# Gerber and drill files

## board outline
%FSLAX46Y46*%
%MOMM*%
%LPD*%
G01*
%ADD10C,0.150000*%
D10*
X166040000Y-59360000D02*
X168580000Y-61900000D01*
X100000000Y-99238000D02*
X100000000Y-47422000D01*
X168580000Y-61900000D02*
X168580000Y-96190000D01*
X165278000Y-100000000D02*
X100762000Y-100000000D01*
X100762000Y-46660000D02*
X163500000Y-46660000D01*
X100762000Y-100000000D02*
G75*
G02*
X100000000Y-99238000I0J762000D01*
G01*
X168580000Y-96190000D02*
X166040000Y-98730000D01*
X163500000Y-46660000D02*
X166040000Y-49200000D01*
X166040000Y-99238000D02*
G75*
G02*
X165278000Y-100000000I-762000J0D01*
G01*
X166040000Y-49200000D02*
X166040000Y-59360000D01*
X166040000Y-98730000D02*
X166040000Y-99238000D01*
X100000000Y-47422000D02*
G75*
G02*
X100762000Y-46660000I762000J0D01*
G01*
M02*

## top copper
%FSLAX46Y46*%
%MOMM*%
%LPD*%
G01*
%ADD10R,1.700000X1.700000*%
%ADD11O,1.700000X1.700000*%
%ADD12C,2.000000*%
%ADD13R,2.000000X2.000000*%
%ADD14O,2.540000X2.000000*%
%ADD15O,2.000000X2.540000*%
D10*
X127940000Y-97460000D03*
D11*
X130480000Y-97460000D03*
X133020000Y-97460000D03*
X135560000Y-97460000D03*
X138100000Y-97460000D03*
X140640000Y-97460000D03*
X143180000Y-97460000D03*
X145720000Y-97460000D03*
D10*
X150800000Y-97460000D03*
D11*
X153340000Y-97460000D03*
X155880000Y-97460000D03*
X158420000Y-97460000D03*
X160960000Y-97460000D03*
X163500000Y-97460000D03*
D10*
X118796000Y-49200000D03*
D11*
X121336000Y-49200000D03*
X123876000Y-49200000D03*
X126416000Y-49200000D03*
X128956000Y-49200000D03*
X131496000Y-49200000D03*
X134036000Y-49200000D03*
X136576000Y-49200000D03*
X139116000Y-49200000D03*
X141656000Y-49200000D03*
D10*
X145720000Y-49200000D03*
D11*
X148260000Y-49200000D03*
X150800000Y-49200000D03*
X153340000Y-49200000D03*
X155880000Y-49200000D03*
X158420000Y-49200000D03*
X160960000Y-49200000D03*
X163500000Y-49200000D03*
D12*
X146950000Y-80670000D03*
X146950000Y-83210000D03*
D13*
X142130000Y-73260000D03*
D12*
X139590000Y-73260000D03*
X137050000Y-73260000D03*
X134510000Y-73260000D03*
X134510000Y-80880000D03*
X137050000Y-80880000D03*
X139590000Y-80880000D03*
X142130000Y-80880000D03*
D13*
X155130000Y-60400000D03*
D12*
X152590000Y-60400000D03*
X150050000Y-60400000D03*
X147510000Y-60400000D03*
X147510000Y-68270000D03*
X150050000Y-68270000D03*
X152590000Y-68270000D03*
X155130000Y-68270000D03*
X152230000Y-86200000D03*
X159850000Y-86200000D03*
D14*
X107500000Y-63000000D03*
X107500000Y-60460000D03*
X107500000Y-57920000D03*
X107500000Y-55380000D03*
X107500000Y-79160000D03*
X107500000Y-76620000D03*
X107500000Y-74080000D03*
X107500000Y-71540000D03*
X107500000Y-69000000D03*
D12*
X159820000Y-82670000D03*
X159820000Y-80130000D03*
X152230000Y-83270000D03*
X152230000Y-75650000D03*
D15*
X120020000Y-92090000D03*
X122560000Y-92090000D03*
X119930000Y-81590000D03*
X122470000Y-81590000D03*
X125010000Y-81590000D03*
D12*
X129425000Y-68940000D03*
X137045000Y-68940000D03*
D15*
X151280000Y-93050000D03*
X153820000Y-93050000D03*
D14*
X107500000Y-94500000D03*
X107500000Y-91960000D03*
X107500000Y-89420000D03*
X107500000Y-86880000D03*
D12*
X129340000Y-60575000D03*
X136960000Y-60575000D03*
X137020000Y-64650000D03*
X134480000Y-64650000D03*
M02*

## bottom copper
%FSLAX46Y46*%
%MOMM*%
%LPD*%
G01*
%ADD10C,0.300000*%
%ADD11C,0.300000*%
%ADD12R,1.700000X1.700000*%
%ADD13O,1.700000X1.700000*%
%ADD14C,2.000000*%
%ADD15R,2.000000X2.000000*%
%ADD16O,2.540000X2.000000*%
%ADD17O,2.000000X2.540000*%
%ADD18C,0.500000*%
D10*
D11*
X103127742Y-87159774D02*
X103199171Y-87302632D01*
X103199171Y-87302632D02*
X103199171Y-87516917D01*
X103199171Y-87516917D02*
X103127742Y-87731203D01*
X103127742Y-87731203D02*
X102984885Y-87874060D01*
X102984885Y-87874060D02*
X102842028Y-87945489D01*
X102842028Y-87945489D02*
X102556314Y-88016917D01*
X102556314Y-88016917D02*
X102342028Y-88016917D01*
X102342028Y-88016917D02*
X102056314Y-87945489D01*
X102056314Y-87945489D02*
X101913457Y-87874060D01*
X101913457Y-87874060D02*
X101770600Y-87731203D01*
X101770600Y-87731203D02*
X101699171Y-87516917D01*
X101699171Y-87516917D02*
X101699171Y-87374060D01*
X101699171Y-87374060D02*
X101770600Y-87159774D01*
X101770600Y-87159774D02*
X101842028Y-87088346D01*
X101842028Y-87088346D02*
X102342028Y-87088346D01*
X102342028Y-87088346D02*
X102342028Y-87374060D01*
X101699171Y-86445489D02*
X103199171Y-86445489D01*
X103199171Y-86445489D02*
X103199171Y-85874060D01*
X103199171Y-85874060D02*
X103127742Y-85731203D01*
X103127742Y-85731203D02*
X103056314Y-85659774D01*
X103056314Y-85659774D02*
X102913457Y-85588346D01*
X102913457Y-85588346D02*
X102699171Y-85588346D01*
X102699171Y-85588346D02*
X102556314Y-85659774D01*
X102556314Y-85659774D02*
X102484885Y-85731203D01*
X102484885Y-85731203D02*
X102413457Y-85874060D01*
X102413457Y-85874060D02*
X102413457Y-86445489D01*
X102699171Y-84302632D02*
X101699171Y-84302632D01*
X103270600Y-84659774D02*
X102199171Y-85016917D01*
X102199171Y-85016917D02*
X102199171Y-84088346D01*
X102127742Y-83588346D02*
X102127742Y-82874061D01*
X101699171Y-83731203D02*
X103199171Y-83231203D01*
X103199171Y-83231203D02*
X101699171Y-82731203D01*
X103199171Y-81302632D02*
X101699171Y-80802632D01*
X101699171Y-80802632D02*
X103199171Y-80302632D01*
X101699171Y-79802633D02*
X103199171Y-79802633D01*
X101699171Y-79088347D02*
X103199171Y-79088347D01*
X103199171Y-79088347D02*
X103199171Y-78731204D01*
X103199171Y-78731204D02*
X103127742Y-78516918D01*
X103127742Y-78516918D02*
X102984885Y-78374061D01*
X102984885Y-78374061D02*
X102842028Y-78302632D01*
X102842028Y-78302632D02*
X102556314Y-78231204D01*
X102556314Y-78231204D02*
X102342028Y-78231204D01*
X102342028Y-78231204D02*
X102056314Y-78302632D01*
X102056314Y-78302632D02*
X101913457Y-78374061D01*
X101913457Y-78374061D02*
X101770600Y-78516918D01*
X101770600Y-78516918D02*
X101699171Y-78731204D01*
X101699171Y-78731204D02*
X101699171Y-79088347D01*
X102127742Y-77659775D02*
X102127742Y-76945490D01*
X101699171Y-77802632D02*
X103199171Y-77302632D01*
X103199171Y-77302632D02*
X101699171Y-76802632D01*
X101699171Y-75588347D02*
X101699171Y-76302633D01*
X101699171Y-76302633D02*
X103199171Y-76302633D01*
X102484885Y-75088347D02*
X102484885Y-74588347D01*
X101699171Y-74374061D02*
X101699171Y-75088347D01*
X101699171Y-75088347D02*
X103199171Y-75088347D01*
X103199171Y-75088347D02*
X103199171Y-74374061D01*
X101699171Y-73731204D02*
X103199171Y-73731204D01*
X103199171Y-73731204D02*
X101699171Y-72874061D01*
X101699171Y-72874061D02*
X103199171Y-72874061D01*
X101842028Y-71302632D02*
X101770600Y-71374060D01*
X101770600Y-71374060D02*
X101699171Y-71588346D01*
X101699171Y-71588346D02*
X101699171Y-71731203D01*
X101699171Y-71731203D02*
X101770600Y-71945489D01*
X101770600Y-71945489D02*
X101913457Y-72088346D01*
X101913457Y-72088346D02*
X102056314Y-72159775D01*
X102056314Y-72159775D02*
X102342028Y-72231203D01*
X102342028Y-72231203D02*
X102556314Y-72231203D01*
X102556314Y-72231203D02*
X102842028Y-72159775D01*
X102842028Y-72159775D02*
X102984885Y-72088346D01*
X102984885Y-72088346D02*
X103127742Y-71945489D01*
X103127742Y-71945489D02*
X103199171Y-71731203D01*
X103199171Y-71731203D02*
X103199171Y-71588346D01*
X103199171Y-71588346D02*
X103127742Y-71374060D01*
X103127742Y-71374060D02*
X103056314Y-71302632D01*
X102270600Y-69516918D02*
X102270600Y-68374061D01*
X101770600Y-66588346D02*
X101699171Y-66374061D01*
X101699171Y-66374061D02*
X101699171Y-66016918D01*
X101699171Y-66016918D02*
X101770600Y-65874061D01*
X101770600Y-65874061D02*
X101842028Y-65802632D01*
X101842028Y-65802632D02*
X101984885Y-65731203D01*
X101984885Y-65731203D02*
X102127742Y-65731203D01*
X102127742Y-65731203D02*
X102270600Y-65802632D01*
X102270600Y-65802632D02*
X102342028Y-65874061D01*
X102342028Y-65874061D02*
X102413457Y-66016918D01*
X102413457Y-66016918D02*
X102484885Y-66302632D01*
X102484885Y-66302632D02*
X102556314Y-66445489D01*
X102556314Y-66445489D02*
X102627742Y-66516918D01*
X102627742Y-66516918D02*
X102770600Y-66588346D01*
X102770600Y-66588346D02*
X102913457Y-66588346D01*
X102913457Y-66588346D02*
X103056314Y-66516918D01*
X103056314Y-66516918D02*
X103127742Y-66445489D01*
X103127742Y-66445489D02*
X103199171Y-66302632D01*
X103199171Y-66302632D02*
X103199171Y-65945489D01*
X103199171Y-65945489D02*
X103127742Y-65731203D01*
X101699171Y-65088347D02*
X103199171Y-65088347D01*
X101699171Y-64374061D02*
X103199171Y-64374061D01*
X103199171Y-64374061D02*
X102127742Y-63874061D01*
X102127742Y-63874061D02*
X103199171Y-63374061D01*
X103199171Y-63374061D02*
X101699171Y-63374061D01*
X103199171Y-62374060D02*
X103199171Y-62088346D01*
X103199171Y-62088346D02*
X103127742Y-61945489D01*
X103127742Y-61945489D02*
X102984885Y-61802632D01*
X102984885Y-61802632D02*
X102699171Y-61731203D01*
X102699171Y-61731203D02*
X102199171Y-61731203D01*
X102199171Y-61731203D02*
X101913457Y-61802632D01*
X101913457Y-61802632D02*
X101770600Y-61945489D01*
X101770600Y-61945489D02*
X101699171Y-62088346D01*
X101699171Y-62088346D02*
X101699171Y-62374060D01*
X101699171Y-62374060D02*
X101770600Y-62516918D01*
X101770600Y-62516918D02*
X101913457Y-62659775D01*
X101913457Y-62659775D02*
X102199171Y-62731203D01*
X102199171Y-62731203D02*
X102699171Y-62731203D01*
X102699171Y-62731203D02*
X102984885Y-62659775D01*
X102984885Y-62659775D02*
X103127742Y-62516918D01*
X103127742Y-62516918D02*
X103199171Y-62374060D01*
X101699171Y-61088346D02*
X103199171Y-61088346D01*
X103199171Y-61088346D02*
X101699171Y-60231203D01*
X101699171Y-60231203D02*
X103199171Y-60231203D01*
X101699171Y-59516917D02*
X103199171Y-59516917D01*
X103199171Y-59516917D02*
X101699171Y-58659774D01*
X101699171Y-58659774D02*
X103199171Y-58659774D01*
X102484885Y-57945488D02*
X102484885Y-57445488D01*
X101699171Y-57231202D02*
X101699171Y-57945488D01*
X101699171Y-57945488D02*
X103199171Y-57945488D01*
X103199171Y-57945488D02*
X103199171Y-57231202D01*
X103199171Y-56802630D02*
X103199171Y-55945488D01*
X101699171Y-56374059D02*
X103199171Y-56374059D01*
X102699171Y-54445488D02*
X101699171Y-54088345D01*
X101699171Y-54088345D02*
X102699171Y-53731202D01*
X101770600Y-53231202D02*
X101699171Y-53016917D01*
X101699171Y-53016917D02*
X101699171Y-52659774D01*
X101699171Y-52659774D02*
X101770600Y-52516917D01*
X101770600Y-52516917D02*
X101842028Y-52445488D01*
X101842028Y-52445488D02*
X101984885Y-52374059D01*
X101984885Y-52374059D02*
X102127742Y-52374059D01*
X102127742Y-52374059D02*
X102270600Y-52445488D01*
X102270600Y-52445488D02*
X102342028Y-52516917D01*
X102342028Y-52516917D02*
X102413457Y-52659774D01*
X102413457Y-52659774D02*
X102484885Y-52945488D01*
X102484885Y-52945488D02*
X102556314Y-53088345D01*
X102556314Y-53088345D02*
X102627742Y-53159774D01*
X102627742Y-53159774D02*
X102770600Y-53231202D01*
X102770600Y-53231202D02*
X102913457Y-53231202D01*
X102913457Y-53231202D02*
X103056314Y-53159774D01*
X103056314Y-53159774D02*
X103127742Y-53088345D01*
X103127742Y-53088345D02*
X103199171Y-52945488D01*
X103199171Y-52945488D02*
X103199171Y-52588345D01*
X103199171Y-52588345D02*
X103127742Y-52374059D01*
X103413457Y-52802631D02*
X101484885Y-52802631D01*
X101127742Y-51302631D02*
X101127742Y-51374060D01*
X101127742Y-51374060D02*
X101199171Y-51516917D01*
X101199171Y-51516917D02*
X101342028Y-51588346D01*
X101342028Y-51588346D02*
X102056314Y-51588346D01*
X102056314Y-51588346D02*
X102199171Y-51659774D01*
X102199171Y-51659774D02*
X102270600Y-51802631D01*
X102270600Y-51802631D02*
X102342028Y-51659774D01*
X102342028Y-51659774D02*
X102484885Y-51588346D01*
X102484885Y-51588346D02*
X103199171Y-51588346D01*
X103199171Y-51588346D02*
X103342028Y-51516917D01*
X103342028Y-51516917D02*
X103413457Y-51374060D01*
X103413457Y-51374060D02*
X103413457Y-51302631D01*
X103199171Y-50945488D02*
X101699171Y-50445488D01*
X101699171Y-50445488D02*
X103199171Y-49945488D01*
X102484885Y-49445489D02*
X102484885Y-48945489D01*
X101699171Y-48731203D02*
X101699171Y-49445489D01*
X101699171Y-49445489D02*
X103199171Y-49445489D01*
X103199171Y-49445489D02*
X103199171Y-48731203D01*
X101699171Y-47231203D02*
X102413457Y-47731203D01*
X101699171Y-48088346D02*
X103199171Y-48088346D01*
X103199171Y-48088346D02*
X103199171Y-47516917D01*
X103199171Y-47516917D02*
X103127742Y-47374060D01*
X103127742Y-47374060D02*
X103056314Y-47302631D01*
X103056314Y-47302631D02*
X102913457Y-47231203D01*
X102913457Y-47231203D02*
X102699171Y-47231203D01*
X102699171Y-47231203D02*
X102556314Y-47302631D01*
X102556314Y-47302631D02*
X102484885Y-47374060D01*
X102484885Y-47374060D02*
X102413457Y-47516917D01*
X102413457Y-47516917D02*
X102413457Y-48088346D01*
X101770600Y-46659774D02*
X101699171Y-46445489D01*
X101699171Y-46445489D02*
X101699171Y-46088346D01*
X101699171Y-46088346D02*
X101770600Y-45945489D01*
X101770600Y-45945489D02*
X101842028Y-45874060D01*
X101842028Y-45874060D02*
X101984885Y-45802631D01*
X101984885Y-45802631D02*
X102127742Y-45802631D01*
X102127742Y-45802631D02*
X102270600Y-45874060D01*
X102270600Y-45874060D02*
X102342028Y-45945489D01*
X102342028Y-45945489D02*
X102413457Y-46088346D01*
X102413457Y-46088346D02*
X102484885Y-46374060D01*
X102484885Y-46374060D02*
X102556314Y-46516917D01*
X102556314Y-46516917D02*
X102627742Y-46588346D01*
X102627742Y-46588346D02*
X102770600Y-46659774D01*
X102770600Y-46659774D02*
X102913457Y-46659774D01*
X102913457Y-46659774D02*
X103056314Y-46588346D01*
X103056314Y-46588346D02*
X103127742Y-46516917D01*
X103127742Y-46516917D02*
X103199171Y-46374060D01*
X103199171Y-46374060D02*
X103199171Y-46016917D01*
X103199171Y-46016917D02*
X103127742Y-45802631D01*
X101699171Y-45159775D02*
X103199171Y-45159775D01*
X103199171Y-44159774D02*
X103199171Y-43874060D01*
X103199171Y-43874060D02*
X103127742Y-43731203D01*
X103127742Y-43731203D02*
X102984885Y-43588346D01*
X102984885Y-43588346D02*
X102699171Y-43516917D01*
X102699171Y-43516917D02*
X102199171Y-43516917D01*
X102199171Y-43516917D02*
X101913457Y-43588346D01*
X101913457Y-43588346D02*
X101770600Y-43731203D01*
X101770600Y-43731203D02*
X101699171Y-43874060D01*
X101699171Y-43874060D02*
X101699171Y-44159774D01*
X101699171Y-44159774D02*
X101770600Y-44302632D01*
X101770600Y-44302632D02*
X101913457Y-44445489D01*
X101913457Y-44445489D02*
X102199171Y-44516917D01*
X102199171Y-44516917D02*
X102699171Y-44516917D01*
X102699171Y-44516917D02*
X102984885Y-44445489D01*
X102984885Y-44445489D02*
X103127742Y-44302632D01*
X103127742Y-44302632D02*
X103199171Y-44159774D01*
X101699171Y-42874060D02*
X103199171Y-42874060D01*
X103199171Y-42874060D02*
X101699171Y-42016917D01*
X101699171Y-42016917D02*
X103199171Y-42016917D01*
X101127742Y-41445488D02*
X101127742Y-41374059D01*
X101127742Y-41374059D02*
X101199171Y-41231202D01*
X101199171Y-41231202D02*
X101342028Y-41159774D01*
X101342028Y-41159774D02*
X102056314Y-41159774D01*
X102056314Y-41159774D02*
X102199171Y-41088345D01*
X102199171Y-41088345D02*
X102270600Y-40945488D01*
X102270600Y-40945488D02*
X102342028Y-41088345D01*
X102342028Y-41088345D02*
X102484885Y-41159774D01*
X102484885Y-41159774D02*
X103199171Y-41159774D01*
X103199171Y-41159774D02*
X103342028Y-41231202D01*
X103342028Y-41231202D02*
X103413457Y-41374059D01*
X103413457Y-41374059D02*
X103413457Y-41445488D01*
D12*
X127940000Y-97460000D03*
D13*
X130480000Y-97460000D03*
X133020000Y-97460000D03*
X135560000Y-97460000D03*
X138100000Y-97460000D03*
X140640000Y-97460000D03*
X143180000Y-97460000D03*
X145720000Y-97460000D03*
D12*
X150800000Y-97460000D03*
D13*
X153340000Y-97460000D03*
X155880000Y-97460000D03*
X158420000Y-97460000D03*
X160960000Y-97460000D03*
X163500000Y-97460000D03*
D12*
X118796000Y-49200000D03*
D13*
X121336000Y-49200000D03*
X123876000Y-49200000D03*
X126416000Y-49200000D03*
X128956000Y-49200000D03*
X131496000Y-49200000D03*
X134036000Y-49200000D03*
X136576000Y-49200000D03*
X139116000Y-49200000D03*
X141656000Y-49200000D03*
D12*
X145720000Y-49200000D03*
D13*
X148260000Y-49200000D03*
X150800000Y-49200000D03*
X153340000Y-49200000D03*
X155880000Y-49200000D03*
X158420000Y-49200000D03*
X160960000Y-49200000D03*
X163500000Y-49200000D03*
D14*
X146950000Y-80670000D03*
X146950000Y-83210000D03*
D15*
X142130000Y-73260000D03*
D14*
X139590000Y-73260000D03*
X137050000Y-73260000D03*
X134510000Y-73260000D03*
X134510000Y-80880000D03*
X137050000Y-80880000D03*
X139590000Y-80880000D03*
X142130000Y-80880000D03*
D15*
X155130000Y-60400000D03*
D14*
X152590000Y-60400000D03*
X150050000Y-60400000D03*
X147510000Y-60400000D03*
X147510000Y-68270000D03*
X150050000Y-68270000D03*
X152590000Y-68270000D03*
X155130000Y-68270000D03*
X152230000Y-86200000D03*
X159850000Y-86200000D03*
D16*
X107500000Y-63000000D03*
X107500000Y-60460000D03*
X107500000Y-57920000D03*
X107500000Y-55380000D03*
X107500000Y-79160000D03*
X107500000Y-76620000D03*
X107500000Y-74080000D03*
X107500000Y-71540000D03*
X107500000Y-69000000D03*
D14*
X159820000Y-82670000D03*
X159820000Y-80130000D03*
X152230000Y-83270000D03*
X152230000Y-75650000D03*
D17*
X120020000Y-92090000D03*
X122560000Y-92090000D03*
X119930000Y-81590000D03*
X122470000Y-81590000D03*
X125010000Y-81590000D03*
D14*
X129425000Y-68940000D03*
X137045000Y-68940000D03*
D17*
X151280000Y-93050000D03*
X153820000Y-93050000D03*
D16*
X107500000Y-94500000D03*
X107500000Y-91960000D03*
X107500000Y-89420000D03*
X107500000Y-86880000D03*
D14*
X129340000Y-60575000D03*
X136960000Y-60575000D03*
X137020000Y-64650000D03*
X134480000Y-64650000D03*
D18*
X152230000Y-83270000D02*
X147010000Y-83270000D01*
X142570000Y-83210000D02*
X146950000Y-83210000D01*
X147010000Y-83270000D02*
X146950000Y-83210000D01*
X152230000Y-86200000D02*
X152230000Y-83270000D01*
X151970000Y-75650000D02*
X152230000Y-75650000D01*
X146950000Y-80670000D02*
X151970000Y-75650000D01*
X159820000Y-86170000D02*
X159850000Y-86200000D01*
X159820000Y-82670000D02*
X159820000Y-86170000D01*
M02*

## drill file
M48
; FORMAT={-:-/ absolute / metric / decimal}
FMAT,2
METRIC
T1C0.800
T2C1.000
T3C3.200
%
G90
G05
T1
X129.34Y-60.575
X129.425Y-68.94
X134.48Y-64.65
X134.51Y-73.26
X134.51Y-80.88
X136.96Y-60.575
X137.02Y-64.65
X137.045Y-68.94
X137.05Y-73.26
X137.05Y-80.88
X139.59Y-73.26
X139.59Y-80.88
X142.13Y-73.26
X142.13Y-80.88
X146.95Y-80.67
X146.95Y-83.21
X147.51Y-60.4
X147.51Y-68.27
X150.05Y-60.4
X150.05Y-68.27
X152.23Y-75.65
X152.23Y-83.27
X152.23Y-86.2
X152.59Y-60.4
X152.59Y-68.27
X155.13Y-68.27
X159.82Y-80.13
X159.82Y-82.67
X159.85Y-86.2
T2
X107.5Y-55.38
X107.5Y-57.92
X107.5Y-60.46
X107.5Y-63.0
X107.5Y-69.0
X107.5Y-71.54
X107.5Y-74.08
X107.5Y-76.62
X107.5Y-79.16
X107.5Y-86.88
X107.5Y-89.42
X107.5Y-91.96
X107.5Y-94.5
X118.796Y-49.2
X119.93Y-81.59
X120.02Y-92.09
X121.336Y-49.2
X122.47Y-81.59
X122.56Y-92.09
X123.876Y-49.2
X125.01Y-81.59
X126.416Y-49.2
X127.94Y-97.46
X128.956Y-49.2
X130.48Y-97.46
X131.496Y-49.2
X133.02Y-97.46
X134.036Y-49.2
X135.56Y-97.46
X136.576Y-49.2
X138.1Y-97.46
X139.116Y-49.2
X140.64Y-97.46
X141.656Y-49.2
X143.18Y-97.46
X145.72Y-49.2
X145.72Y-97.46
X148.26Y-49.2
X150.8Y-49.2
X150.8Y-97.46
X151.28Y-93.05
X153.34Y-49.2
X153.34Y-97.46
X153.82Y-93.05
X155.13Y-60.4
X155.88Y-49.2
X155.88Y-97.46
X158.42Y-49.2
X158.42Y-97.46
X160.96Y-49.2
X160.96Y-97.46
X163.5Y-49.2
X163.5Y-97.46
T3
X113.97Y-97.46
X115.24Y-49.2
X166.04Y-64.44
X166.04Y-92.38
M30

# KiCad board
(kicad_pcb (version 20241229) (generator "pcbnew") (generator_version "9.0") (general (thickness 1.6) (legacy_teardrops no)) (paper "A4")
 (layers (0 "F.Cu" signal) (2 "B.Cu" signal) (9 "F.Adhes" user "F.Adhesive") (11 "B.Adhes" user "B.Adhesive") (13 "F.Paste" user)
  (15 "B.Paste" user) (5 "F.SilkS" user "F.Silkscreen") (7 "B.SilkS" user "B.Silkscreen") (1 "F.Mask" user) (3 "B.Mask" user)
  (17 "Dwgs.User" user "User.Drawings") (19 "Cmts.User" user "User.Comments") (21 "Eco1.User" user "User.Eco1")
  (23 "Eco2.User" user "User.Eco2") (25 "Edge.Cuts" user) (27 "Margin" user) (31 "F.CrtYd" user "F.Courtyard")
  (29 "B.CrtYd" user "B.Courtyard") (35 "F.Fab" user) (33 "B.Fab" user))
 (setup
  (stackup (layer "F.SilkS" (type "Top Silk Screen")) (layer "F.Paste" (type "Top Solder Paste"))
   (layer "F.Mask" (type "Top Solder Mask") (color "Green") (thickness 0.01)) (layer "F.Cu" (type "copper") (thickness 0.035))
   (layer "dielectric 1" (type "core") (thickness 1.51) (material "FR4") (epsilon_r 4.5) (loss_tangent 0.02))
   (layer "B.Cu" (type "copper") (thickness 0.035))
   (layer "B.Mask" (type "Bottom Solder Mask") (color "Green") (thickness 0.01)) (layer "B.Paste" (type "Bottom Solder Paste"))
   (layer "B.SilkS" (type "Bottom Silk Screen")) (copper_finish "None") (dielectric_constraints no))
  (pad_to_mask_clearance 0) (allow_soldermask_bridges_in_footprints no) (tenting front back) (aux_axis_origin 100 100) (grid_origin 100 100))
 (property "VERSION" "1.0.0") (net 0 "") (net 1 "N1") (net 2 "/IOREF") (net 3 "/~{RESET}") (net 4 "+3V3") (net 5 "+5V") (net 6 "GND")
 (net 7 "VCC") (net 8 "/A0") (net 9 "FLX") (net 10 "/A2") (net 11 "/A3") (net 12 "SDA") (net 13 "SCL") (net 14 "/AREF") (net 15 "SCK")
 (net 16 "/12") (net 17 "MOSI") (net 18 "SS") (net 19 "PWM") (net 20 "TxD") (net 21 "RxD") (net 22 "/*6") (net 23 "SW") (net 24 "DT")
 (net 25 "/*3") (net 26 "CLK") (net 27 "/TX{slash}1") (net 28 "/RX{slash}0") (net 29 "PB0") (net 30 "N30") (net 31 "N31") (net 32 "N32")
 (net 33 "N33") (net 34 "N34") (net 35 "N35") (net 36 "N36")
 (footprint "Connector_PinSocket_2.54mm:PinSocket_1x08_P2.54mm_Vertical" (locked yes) (layer "F.Cu") (at 127.94 97.46 90)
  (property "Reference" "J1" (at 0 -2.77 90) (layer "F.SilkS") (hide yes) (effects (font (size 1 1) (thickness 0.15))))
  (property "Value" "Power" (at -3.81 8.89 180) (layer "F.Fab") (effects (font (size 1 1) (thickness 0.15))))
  (pad "1" thru_hole rect (at 0 0 90) (size 1.7 1.7) (drill 1) (layers "*.Cu" "*.Mask") (remove_unused_layers no) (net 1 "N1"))
  (pad "2" thru_hole oval (at 0 2.54 90) (size 1.7 1.7) (drill 1) (layers "*.Cu" "*.Mask") (remove_unused_layers no) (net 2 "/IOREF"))
  (pad "3" thru_hole oval (at 0 5.08 90) (size 1.7 1.7) (drill 1) (layers "*.Cu" "*.Mask") (remove_unused_layers no) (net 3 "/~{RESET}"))
  (pad "4" thru_hole oval (at 0 7.62 90) (size 1.7 1.7) (drill 1) (layers "*.Cu" "*.Mask") (remove_unused_layers no) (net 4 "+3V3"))
  (pad "5" thru_hole oval (at 0 10.16 90) (size 1.7 1.7) (drill 1) (layers "*.Cu" "*.Mask") (remove_unused_layers no) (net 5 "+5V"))
  (pad "6" thru_hole oval (at 0 12.7 90) (size 1.7 1.7) (drill 1) (layers "*.Cu" "*.Mask") (remove_unused_layers no) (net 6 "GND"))
  (pad "7" thru_hole oval (at 0 15.24 90) (size 1.7 1.7) (drill 1) (layers "*.Cu" "*.Mask") (remove_unused_layers no) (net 6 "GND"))
  (pad "8" thru_hole oval (at 0 17.78 90) (size 1.7 1.7) (drill 1) (layers "*.Cu" "*.Mask") (remove_unused_layers no) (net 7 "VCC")))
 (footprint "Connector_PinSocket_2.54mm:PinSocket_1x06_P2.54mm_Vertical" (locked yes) (layer "F.Cu") (at 150.8 97.46 90)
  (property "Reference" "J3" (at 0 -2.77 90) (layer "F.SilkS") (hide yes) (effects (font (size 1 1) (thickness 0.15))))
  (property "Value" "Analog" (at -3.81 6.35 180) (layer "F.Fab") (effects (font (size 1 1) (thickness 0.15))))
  (pad "1" thru_hole rect (at 0 0 90) (size 1.7 1.7) (drill 1) (layers "*.Cu" "*.Mask") (remove_unused_layers no) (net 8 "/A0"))
  (pad "2" thru_hole oval (at 0 2.54 90) (size 1.7 1.7) (drill 1) (layers "*.Cu" "*.Mask") (remove_unused_layers no) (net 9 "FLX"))
  (pad "3" thru_hole oval (at 0 5.08 90) (size 1.7 1.7) (drill 1) (layers "*.Cu" "*.Mask") (remove_unused_layers no) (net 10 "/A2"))
  (pad "4" thru_hole oval (at 0 7.62 90) (size 1.7 1.7) (drill 1) (layers "*.Cu" "*.Mask") (remove_unused_layers no) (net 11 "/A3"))
  (pad "5" thru_hole oval (at 0 10.16 90) (size 1.7 1.7) (drill 1) (layers "*.Cu" "*.Mask") (remove_unused_layers no) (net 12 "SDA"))
  (pad "6" thru_hole oval (at 0 12.7 90) (size 1.7 1.7) (drill 1) (layers "*.Cu" "*.Mask") (remove_unused_layers no) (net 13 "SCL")))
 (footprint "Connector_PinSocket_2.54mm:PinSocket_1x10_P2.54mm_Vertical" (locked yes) (layer "F.Cu") (at 118.796 49.2 90)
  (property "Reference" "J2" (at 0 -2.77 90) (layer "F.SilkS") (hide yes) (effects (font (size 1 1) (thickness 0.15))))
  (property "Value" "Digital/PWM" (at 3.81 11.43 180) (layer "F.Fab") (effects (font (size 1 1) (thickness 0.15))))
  (pad "1" thru_hole rect (at 0 0 90) (size 1.7 1.7) (drill 1) (layers "*.Cu" "*.Mask") (remove_unused_layers no) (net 13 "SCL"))
  (pad "2" thru_hole oval (at 0 2.54 90) (size 1.7 1.7) (drill 1) (layers "*.Cu" "*.Mask") (remove_unused_layers no) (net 12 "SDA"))
  (pad "3" thru_hole oval (at 0 5.08 90) (size 1.7 1.7) (drill 1) (layers "*.Cu" "*.Mask") (remove_unused_layers no) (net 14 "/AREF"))
  (pad "4" thru_hole oval (at 0 7.62 90) (size 1.7 1.7) (drill 1) (layers "*.Cu" "*.Mask") (remove_unused_layers no) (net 6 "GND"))
  (pad "5" thru_hole oval (at 0 10.16 90) (size 1.7 1.7) (drill 1) (layers "*.Cu" "*.Mask") (remove_unused_layers no) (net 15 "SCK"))
  (pad "6" thru_hole oval (at 0 12.7 90) (size 1.7 1.7) (drill 1) (layers "*.Cu" "*.Mask") (remove_unused_layers no) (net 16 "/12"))
  (pad "7" thru_hole oval (at 0 15.24 90) (size 1.7 1.7) (drill 1) (layers "*.Cu" "*.Mask") (remove_unused_layers no) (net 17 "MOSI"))
  (pad "8" thru_hole oval (at 0 17.78 90) (size 1.7 1.7) (drill 1) (layers "*.Cu" "*.Mask") (remove_unused_layers no) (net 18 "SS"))
  (pad "9" thru_hole oval (at 0 20.32 90) (size 1.7 1.7) (drill 1) (layers "*.Cu" "*.Mask") (remove_unused_layers no) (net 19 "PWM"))
  (pad "10" thru_hole oval (at 0 22.86 90) (size 1.7 1.7) (drill 1) (layers "*.Cu" "*.Mask") (remove_unused_layers no) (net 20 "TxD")))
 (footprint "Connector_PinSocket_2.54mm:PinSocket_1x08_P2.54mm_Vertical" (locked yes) (layer "F.Cu") (at 145.72 49.2 90)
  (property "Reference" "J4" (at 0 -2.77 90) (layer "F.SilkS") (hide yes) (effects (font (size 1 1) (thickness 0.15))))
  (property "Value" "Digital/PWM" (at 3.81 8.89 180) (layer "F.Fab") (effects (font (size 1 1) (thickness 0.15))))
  (pad "1" thru_hole rect (at 0 0 90) (size 1.7 1.7) (drill 1) (layers "*.Cu" "*.Mask") (remove_unused_layers no) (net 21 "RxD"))
  (pad "2" thru_hole oval (at 0 2.54 90) (size 1.7 1.7) (drill 1) (layers "*.Cu" "*.Mask") (remove_unused_layers no) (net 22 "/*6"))
  (pad "3" thru_hole oval (at 0 5.08 90) (size 1.7 1.7) (drill 1) (layers "*.Cu" "*.Mask") (remove_unused_layers no) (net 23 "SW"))
  (pad "4" thru_hole oval (at 0 7.62 90) (size 1.7 1.7) (drill 1) (layers "*.Cu" "*.Mask") (remove_unused_layers no) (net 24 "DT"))
  (pad "5" thru_hole oval (at 0 10.16 90) (size 1.7 1.7) (drill 1) (layers "*.Cu" "*.Mask") (remove_unused_layers no) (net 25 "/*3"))
  (pad "6" thru_hole oval (at 0 12.7 90) (size 1.7 1.7) (drill 1) (layers "*.Cu" "*.Mask") (remove_unused_layers no) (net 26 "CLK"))
  (pad "7" thru_hole oval (at 0 15.24 90) (size 1.7 1.7) (drill 1) (layers "*.Cu" "*.Mask") (remove_unused_layers no) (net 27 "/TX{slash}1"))
  (pad "8" thru_hole oval (at 0 17.78 90) (size 1.7 1.7) (drill 1) (layers "*.Cu" "*.Mask") (remove_unused_layers no) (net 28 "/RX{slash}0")))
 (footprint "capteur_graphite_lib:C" (layer "F.Cu") (at 146.95 81.94 -90)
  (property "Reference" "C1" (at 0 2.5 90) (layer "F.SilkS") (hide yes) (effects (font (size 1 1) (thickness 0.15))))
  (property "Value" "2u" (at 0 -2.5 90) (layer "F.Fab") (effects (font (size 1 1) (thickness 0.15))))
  (pad "1" thru_hole circle (at -1.27 0 270) (size 2 2) (drill 0.8) (layers "*.Cu" "*.Mask") (remove_unused_layers no) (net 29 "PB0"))
  (pad "2" thru_hole circle (at 1.27 0 270) (size 2 2) (drill 0.8) (layers "*.Cu" "*.Mask") (remove_unused_layers no) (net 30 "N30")))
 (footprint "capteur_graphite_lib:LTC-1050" (layer "F.Cu") (at 134.51 80.88 -90)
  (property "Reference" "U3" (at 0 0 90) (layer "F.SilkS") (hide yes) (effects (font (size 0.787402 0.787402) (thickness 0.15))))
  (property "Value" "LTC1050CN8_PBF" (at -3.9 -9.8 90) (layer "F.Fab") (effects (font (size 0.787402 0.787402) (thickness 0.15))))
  (pad "1" thru_hole rect (at -7.62 -7.62 270) (size 2 2) (drill 0.8) (layers "*.Cu" "*.Mask") (remove_unused_layers no) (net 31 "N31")
   (solder_mask_margin 0.102))
  (pad "2" thru_hole circle (at -7.62 -5.08 270) (size 2 2) (drill 0.8) (layers "*.Cu" "*.Mask") (remove_unused_layers no) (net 29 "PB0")
   (solder_mask_margin 0.102))
  (pad "3" thru_hole circle (at -7.62 -2.54 270) (size 2 2) (drill 0.8) (layers "*.Cu" "*.Mask") (remove_unused_layers no) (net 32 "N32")
   (solder_mask_margin 0.102))
  (pad "4" thru_hole circle (at -7.62 0 270) (size 2 2) (drill 0.8) (layers "*.Cu" "*.Mask") (remove_unused_layers no) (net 6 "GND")
   (solder_mask_margin 0.102))
  (pad "5" thru_hole circle (at 0 0 270) (size 2 2) (drill 0.8) (layers "*.Cu" "*.Mask") (remove_unused_layers no) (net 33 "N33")
   (solder_mask_margin 0.102))
  (pad "6" thru_hole circle (at 0 -2.54 270) (size 2 2) (drill 0.8) (layers "*.Cu" "*.Mask") (remove_unused_layers no) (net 30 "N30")
   (solder_mask_margin 0.102))
  (pad "7" thru_hole circle (at 0 -5.08 270) (size 2 2) (drill 0.8) (layers "*.Cu" "*.Mask") (remove_unused_layers no) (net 7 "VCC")
   (solder_mask_margin 0.102))
  (pad "8" thru_hole circle (at 0 -7.62 270) (size 2 2) (drill 0.8) (layers "*.Cu" "*.Mask") (remove_unused_layers no) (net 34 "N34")
   (solder_mask_margin 0.102)))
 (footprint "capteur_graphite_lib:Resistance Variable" (layer "F.Cu") (at 151.32 64.335 -90)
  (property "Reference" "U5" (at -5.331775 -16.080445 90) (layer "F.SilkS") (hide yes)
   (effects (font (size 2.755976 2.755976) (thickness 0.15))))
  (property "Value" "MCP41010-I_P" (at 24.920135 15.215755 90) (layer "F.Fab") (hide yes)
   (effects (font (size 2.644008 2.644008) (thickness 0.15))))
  (pad "1" thru_hole rect (at -3.935 -3.81 270) (size 2 2) (drill 1) (layers "*.Cu" "*.Mask") (remove_unused_layers no) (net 18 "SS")
   (solder_mask_margin 0.102))
  (pad "2" thru_hole circle (at -3.935 -1.27 270) (size 2 2) (drill 0.8) (layers "*.Cu" "*.Mask") (remove_unused_layers no) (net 15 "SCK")
   (solder_mask_margin 0.102))
  (pad "3" thru_hole circle (at -3.935 1.27 270) (size 2 2) (drill 0.8) (layers "*.Cu" "*.Mask") (remove_unused_layers no) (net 17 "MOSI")
   (solder_mask_margin 0.102))
  (pad "4" thru_hole circle (at -3.935 3.81 270) (size 2 2) (drill 0.8) (layers "*.Cu" "*.Mask") (remove_unused_layers no) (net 6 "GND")
   (solder_mask_margin 0.102))
  (pad "5" thru_hole circle (at 3.935 3.81 270) (size 2 2) (drill 0.8) (layers "*.Cu" "*.Mask") (remove_unused_layers no) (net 6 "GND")
   (solder_mask_margin 0.102))
  (pad "6" thru_hole circle (at 3.935 1.27 270) (size 2 2) (drill 0.8) (layers "*.Cu" "*.Mask") (remove_unused_layers no) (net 6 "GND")
   (solder_mask_margin 0.102))
  (pad "7" thru_hole circle (at 3.935 -1.27 270) (size 2 2) (drill 0.8) (layers "*.Cu" "*.Mask") (remove_unused_layers no) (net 29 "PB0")
   (solder_mask_margin 0.102))
  (pad "8" thru_hole circle (at 3.935 -3.81 270) (size 2 2) (drill 0.8) (layers "*.Cu" "*.Mask") (remove_unused_layers no) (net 7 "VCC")
   (solder_mask_margin 0.102)))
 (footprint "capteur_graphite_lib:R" (layer "F.Cu") (at 152.23 86.2)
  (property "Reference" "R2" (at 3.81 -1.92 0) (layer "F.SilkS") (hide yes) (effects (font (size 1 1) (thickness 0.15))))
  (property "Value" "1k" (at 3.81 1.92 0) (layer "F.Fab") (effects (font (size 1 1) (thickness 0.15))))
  (pad "1" thru_hole circle (at 0 0) (size 2 2) (drill 0.8) (layers "*.Cu" "*.Mask") (remove_unused_layers no) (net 30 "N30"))
  (pad "2" thru_hole circle (at 7.62 0) (size 2 2) (drill 0.8) (layers "*.Cu" "*.Mask") (remove_unused_layers no) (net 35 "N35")))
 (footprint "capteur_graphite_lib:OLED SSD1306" (layer "F.Cu") (at 107.5 59.19 90)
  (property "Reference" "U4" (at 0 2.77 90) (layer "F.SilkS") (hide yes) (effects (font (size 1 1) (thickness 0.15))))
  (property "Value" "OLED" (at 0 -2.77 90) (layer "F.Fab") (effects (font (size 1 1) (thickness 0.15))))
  (pad "1" thru_hole oval (at -3.81 0 90) (size 2 2.54) (drill 1) (layers "*.Cu" "*.Mask") (remove_unused_layers no) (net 6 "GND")
   (thermal_bridge_angle 45))
  (pad "2" thru_hole oval (at -1.27 0 90) (size 2 2.54) (drill 1) (layers "*.Cu" "*.Mask") (remove_unused_layers no) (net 7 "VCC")
   (thermal_bridge_angle 45))
  (pad "3" thru_hole oval (at 1.27 0 90) (size 2 2.54) (drill 1) (layers "*.Cu" "*.Mask") (remove_unused_layers no) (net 13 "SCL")
   (thermal_bridge_angle 45))
  (pad "4" thru_hole oval (at 3.81 0 90) (size 2 2.54) (drill 1) (layers "*.Cu" "*.Mask") (remove_unused_layers no) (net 12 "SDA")
   (thermal_bridge_angle 45)))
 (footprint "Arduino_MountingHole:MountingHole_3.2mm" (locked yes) (layer "F.Cu") (at 115.24 49.2)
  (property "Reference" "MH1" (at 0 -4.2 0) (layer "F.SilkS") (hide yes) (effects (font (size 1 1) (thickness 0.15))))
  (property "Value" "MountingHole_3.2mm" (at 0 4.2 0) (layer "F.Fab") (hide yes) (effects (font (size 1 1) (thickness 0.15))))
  (pad "" np_thru_hole circle (at 0 0) (size 3.2 3.2) (drill 3.2) (layers "*.Cu" "*.Mask")))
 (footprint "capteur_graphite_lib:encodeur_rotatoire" (layer "F.Cu") (at 107.5 74.08 90)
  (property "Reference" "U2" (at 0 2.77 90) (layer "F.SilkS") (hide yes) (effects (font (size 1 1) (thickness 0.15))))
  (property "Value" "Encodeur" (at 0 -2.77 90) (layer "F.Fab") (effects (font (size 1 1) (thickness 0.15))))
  (pad "1" thru_hole oval (at -5.08 0 90) (size 2 2.54) (drill 1) (layers "*.Cu" "*.Mask") (remove_unused_layers no) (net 6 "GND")
   (thermal_bridge_angle 45))
  (pad "2" thru_hole oval (at -2.54 0 90) (size 2 2.54) (drill 1) (layers "*.Cu" "*.Mask") (remove_unused_layers no) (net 7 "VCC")
   (thermal_bridge_angle 45))
  (pad "3" thru_hole oval (at 0 0 90) (size 2 2.54) (drill 1) (layers "*.Cu" "*.Mask") (remove_unused_layers no) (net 23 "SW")
   (thermal_bridge_angle 45))
  (pad "4" thru_hole oval (at 2.54 0 90) (size 2 2.54) (drill 1) (layers "*.Cu" "*.Mask") (remove_unused_layers no) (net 24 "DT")
   (thermal_bridge_angle 45))
  (pad "5" thru_hole oval (at 5.08 0 90) (size 2 2.54) (drill 1) (layers "*.Cu" "*.Mask") (remove_unused_layers no) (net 26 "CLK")
   (thermal_bridge_angle 45)))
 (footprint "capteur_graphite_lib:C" (layer "F.Cu") (at 159.82 81.4 90)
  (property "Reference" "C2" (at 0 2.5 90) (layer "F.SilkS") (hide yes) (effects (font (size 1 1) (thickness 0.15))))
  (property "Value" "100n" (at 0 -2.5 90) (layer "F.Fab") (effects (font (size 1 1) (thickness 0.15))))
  (pad "1" thru_hole circle (at -1.27 0 90) (size 2 2) (drill 0.8) (layers "*.Cu" "*.Mask") (remove_unused_layers no) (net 35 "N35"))
  (pad "2" thru_hole circle (at 1.27 0 90) (size 2 2) (drill 0.8) (layers "*.Cu" "*.Mask") (remove_unused_layers no) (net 6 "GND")))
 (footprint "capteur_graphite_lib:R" (layer "F.Cu") (at 152.23 83.27 90)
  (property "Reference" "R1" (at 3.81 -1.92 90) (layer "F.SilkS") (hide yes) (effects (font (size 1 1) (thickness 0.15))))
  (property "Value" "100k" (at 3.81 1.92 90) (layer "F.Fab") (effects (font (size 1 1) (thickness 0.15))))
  (pad "1" thru_hole circle (at 0 0 90) (size 2 2) (drill 0.8) (layers "*.Cu" "*.Mask") (remove_unused_layers no) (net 30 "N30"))
  (pad "2" thru_hole circle (at 7.62 0 90) (size 2 2) (drill 0.8) (layers "*.Cu" "*.Mask") (remove_unused_layers no) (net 29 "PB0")))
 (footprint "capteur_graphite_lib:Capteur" (layer "F.Cu") (at 121.29 92.09)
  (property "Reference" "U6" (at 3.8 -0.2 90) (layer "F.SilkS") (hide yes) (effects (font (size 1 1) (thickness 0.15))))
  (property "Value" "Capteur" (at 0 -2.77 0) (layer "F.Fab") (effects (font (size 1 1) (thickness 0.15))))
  (pad "1" thru_hole oval (at -1.27 0) (size 2 2.54) (drill 1) (layers "*.Cu" "*.Mask") (remove_unused_layers no) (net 7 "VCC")
   (thermal_bridge_angle 45))
  (pad "2" thru_hole oval (at 1.27 0) (size 2 2.54) (drill 1) (layers "*.Cu" "*.Mask") (remove_unused_layers no) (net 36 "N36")
   (thermal_bridge_angle 45)))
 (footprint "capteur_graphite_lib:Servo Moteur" (layer "F.Cu") (at 122.47 81.59)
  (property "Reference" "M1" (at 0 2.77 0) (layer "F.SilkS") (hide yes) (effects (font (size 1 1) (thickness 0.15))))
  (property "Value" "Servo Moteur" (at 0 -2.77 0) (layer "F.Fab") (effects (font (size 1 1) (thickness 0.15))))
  (pad "1" thru_hole oval (at -2.54 0) (size 2 2.54) (drill 1) (layers "*.Cu" "*.Mask") (remove_unused_layers no) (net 19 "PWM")
   (thermal_bridge_angle 45))
  (pad "2" thru_hole oval (at 0 0) (size 2 2.54) (drill 1) (layers "*.Cu" "*.Mask") (remove_unused_layers no) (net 7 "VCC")
   (thermal_bridge_angle 45))
  (pad "3" thru_hole oval (at 2.54 0) (size 2 2.54) (drill 1) (layers "*.Cu" "*.Mask") (remove_unused_layers no) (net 6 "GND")
   (thermal_bridge_angle 45)))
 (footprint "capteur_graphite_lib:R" (layer "F.Cu") (at 129.425 68.94)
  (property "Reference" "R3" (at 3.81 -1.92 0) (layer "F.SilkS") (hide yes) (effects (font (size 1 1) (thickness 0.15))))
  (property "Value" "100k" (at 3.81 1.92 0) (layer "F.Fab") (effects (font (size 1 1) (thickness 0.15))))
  (pad "1" thru_hole circle (at 0 0) (size 2 2) (drill 0.8) (layers "*.Cu" "*.Mask") (remove_unused_layers no) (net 6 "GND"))
  (pad "2" thru_hole circle (at 7.62 0) (size 2 2) (drill 0.8) (layers "*.Cu" "*.Mask") (remove_unused_layers no) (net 32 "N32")))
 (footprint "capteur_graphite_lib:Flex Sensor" (layer "F.Cu") (at 152.55 93.05)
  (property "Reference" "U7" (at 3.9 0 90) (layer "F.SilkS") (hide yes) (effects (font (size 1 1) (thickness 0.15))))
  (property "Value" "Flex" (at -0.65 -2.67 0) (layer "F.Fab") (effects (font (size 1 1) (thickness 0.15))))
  (pad "1" thru_hole oval (at -1.27 0) (size 2 2.54) (drill 1) (layers "*.Cu" "*.Mask") (remove_unused_layers no) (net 7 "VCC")
   (thermal_bridge_angle 45))
  (pad "2" thru_hole oval (at 1.27 0) (size 2 2.54) (drill 1) (layers "*.Cu" "*.Mask") (remove_unused_layers no) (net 9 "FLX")
   (thermal_bridge_angle 45)))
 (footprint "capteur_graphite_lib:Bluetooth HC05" (layer "F.Cu") (at 107.5 90.69 90)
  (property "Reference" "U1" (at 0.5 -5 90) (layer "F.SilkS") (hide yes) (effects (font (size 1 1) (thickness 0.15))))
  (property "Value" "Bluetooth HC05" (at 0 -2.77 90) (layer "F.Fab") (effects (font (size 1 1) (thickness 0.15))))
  (pad "1" thru_hole oval (at -3.81 0 90) (size 2 2.54) (drill 1) (layers "*.Cu" "*.Mask") (remove_unused_layers no) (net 7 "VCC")
   (thermal_bridge_angle 45))
  (pad "2" thru_hole oval (at -1.27 0 90) (size 2 2.54) (drill 1) (layers "*.Cu" "*.Mask") (remove_unused_layers no) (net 6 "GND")
   (thermal_bridge_angle 45))
  (pad "3" thru_hole oval (at 1.27 0 90) (size 2 2.54) (drill 1) (layers "*.Cu" "*.Mask") (remove_unused_layers no) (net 20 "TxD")
   (thermal_bridge_angle 45))
  (pad "4" thru_hole oval (at 3.81 0 90) (size 2 2.54) (drill 1) (layers "*.Cu" "*.Mask") (remove_unused_layers no) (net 21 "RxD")
   (thermal_bridge_angle 45)))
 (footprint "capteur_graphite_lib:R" (layer "F.Cu") (at 129.34 60.575)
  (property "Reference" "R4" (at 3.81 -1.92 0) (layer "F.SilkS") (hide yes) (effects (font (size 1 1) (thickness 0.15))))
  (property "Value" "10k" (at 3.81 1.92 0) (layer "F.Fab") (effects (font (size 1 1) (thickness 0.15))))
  (pad "1" thru_hole circle (at 0 0) (size 2 2) (drill 0.8) (layers "*.Cu" "*.Mask") (remove_unused_layers no) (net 32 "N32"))
  (pad "2" thru_hole circle (at 7.62 0) (size 2 2) (drill 0.8) (layers "*.Cu" "*.Mask") (remove_unused_layers no) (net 36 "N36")))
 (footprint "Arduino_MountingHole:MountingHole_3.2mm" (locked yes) (layer "F.Cu") (at 113.97 97.46)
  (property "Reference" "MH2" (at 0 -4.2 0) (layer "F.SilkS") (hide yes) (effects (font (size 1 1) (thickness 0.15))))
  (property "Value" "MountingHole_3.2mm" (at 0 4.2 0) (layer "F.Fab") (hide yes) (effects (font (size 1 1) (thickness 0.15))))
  (pad "" np_thru_hole circle (at 0 0) (size 3.2 3.2) (drill 3.2) (layers "*.Cu" "*.Mask")))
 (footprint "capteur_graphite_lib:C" (layer "F.Cu") (at 135.75 64.65 180)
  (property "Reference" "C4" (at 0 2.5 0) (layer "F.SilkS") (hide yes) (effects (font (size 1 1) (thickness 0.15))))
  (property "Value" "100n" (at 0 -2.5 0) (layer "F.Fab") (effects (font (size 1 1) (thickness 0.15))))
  (pad "1" thru_hole circle (at -1.27 0 180) (size 2 2) (drill 0.8) (layers "*.Cu" "*.Mask") (remove_unused_layers no) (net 32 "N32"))
  (pad "2" thru_hole circle (at 1.27 0 180) (size 2 2) (drill 0.8) (layers "*.Cu" "*.Mask") (remove_unused_layers no) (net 6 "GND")))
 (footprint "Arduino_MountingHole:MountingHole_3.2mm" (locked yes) (layer "F.Cu") (at 166.04 64.44)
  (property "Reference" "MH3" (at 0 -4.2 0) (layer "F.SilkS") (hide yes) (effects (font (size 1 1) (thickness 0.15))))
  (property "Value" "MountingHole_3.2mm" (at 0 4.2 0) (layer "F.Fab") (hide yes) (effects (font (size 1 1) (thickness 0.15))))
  (pad "" np_thru_hole circle (at 0 0) (size 3.2 3.2) (drill 3.2) (layers "*.Cu" "*.Mask")))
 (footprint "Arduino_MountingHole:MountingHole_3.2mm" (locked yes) (layer "F.Cu") (at 166.04 92.38)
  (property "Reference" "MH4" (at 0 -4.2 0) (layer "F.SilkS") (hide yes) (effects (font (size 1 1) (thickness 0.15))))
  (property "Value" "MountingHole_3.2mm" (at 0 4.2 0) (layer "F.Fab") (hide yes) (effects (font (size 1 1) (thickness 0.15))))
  (pad "" np_thru_hole circle (at 0 0) (size 3.2 3.2) (drill 3.2) (layers "*.Cu" "*.Mask")))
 (gr_line (start 166.04 59.36) (end 168.58 61.9) (stroke (width 0.15) (type solid)) (layer "Edge.Cuts"))
 (gr_line (start 100 99.238) (end 100 47.422) (stroke (width 0.15) (type solid)) (layer "Edge.Cuts"))
 (gr_line (start 168.58 61.9) (end 168.58 96.19) (stroke (width 0.15) (type solid)) (layer "Edge.Cuts"))
 (gr_line (start 165.278 100) (end 100.762 100) (stroke (width 0.15) (type solid)) (layer "Edge.Cuts"))
 (gr_line (start 100.762 46.66) (end 163.5 46.66) (stroke (width 0.15) (type solid)) (layer "Edge.Cuts"))
 (gr_arc (start 100.762 100) (mid 100.223185 99.776815) (end 100 99.238) (stroke (width 0.15) (type solid)) (layer "Edge.Cuts"))
 (gr_line (start 168.58 96.19) (end 166.04 98.73) (stroke (width 0.15) (type solid)) (layer "Edge.Cuts"))
 (gr_line (start 163.5 46.66) (end 166.04 49.2) (stroke (width 0.15) (type solid)) (layer "Edge.Cuts"))
 (gr_arc (start 166.04 99.238) (mid 165.816815 99.776815) (end 165.278 100) (stroke (width 0.15) (type solid)) (layer "Edge.Cuts"))
 (gr_line (start 166.04 49.2) (end 166.04 59.36) (stroke (width 0.15) (type solid)) (layer "Edge.Cuts"))
 (gr_line (start 166.04 98.73) (end 166.04 99.238) (stroke (width 0.15) (type solid)) (layer "Edge.Cuts"))
 (gr_arc (start 100 47.422) (mid 100.223185 46.883185) (end 100.762 46.66) (stroke (width 0.15) (type solid)) (layer "Edge.Cuts"))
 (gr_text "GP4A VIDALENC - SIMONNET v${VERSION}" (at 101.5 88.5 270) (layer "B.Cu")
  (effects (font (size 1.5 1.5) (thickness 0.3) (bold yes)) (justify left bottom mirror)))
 (segment (start 152.23 83.27) (end 147.01 83.27) (width 0.5) (layer "B.Cu") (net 30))
 (segment (start 142.57 83.21) (end 146.95 83.21) (width 0.5) (layer "B.Cu") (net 30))
 (segment (start 147.01 83.27) (end 146.95 83.21) (width 0.5) (layer "B.Cu") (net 30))
 (segment (start 152.23 86.2) (end 152.23 83.27) (width 0.5) (layer "B.Cu") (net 30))
 (segment (start 151.97 75.65) (end 152.23 75.65) (width 0.5) (layer "B.Cu") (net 29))
 (segment (start 146.95 80.67) (end 151.97 75.65) (width 0.5) (layer "B.Cu") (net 29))
 (segment (start 159.82 86.17) (end 159.85 86.2) (width 0.5) (layer "B.Cu") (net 35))
 (segment (start 159.82 82.67) (end 159.82 86.17) (width 0.5) (layer "B.Cu") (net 35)))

